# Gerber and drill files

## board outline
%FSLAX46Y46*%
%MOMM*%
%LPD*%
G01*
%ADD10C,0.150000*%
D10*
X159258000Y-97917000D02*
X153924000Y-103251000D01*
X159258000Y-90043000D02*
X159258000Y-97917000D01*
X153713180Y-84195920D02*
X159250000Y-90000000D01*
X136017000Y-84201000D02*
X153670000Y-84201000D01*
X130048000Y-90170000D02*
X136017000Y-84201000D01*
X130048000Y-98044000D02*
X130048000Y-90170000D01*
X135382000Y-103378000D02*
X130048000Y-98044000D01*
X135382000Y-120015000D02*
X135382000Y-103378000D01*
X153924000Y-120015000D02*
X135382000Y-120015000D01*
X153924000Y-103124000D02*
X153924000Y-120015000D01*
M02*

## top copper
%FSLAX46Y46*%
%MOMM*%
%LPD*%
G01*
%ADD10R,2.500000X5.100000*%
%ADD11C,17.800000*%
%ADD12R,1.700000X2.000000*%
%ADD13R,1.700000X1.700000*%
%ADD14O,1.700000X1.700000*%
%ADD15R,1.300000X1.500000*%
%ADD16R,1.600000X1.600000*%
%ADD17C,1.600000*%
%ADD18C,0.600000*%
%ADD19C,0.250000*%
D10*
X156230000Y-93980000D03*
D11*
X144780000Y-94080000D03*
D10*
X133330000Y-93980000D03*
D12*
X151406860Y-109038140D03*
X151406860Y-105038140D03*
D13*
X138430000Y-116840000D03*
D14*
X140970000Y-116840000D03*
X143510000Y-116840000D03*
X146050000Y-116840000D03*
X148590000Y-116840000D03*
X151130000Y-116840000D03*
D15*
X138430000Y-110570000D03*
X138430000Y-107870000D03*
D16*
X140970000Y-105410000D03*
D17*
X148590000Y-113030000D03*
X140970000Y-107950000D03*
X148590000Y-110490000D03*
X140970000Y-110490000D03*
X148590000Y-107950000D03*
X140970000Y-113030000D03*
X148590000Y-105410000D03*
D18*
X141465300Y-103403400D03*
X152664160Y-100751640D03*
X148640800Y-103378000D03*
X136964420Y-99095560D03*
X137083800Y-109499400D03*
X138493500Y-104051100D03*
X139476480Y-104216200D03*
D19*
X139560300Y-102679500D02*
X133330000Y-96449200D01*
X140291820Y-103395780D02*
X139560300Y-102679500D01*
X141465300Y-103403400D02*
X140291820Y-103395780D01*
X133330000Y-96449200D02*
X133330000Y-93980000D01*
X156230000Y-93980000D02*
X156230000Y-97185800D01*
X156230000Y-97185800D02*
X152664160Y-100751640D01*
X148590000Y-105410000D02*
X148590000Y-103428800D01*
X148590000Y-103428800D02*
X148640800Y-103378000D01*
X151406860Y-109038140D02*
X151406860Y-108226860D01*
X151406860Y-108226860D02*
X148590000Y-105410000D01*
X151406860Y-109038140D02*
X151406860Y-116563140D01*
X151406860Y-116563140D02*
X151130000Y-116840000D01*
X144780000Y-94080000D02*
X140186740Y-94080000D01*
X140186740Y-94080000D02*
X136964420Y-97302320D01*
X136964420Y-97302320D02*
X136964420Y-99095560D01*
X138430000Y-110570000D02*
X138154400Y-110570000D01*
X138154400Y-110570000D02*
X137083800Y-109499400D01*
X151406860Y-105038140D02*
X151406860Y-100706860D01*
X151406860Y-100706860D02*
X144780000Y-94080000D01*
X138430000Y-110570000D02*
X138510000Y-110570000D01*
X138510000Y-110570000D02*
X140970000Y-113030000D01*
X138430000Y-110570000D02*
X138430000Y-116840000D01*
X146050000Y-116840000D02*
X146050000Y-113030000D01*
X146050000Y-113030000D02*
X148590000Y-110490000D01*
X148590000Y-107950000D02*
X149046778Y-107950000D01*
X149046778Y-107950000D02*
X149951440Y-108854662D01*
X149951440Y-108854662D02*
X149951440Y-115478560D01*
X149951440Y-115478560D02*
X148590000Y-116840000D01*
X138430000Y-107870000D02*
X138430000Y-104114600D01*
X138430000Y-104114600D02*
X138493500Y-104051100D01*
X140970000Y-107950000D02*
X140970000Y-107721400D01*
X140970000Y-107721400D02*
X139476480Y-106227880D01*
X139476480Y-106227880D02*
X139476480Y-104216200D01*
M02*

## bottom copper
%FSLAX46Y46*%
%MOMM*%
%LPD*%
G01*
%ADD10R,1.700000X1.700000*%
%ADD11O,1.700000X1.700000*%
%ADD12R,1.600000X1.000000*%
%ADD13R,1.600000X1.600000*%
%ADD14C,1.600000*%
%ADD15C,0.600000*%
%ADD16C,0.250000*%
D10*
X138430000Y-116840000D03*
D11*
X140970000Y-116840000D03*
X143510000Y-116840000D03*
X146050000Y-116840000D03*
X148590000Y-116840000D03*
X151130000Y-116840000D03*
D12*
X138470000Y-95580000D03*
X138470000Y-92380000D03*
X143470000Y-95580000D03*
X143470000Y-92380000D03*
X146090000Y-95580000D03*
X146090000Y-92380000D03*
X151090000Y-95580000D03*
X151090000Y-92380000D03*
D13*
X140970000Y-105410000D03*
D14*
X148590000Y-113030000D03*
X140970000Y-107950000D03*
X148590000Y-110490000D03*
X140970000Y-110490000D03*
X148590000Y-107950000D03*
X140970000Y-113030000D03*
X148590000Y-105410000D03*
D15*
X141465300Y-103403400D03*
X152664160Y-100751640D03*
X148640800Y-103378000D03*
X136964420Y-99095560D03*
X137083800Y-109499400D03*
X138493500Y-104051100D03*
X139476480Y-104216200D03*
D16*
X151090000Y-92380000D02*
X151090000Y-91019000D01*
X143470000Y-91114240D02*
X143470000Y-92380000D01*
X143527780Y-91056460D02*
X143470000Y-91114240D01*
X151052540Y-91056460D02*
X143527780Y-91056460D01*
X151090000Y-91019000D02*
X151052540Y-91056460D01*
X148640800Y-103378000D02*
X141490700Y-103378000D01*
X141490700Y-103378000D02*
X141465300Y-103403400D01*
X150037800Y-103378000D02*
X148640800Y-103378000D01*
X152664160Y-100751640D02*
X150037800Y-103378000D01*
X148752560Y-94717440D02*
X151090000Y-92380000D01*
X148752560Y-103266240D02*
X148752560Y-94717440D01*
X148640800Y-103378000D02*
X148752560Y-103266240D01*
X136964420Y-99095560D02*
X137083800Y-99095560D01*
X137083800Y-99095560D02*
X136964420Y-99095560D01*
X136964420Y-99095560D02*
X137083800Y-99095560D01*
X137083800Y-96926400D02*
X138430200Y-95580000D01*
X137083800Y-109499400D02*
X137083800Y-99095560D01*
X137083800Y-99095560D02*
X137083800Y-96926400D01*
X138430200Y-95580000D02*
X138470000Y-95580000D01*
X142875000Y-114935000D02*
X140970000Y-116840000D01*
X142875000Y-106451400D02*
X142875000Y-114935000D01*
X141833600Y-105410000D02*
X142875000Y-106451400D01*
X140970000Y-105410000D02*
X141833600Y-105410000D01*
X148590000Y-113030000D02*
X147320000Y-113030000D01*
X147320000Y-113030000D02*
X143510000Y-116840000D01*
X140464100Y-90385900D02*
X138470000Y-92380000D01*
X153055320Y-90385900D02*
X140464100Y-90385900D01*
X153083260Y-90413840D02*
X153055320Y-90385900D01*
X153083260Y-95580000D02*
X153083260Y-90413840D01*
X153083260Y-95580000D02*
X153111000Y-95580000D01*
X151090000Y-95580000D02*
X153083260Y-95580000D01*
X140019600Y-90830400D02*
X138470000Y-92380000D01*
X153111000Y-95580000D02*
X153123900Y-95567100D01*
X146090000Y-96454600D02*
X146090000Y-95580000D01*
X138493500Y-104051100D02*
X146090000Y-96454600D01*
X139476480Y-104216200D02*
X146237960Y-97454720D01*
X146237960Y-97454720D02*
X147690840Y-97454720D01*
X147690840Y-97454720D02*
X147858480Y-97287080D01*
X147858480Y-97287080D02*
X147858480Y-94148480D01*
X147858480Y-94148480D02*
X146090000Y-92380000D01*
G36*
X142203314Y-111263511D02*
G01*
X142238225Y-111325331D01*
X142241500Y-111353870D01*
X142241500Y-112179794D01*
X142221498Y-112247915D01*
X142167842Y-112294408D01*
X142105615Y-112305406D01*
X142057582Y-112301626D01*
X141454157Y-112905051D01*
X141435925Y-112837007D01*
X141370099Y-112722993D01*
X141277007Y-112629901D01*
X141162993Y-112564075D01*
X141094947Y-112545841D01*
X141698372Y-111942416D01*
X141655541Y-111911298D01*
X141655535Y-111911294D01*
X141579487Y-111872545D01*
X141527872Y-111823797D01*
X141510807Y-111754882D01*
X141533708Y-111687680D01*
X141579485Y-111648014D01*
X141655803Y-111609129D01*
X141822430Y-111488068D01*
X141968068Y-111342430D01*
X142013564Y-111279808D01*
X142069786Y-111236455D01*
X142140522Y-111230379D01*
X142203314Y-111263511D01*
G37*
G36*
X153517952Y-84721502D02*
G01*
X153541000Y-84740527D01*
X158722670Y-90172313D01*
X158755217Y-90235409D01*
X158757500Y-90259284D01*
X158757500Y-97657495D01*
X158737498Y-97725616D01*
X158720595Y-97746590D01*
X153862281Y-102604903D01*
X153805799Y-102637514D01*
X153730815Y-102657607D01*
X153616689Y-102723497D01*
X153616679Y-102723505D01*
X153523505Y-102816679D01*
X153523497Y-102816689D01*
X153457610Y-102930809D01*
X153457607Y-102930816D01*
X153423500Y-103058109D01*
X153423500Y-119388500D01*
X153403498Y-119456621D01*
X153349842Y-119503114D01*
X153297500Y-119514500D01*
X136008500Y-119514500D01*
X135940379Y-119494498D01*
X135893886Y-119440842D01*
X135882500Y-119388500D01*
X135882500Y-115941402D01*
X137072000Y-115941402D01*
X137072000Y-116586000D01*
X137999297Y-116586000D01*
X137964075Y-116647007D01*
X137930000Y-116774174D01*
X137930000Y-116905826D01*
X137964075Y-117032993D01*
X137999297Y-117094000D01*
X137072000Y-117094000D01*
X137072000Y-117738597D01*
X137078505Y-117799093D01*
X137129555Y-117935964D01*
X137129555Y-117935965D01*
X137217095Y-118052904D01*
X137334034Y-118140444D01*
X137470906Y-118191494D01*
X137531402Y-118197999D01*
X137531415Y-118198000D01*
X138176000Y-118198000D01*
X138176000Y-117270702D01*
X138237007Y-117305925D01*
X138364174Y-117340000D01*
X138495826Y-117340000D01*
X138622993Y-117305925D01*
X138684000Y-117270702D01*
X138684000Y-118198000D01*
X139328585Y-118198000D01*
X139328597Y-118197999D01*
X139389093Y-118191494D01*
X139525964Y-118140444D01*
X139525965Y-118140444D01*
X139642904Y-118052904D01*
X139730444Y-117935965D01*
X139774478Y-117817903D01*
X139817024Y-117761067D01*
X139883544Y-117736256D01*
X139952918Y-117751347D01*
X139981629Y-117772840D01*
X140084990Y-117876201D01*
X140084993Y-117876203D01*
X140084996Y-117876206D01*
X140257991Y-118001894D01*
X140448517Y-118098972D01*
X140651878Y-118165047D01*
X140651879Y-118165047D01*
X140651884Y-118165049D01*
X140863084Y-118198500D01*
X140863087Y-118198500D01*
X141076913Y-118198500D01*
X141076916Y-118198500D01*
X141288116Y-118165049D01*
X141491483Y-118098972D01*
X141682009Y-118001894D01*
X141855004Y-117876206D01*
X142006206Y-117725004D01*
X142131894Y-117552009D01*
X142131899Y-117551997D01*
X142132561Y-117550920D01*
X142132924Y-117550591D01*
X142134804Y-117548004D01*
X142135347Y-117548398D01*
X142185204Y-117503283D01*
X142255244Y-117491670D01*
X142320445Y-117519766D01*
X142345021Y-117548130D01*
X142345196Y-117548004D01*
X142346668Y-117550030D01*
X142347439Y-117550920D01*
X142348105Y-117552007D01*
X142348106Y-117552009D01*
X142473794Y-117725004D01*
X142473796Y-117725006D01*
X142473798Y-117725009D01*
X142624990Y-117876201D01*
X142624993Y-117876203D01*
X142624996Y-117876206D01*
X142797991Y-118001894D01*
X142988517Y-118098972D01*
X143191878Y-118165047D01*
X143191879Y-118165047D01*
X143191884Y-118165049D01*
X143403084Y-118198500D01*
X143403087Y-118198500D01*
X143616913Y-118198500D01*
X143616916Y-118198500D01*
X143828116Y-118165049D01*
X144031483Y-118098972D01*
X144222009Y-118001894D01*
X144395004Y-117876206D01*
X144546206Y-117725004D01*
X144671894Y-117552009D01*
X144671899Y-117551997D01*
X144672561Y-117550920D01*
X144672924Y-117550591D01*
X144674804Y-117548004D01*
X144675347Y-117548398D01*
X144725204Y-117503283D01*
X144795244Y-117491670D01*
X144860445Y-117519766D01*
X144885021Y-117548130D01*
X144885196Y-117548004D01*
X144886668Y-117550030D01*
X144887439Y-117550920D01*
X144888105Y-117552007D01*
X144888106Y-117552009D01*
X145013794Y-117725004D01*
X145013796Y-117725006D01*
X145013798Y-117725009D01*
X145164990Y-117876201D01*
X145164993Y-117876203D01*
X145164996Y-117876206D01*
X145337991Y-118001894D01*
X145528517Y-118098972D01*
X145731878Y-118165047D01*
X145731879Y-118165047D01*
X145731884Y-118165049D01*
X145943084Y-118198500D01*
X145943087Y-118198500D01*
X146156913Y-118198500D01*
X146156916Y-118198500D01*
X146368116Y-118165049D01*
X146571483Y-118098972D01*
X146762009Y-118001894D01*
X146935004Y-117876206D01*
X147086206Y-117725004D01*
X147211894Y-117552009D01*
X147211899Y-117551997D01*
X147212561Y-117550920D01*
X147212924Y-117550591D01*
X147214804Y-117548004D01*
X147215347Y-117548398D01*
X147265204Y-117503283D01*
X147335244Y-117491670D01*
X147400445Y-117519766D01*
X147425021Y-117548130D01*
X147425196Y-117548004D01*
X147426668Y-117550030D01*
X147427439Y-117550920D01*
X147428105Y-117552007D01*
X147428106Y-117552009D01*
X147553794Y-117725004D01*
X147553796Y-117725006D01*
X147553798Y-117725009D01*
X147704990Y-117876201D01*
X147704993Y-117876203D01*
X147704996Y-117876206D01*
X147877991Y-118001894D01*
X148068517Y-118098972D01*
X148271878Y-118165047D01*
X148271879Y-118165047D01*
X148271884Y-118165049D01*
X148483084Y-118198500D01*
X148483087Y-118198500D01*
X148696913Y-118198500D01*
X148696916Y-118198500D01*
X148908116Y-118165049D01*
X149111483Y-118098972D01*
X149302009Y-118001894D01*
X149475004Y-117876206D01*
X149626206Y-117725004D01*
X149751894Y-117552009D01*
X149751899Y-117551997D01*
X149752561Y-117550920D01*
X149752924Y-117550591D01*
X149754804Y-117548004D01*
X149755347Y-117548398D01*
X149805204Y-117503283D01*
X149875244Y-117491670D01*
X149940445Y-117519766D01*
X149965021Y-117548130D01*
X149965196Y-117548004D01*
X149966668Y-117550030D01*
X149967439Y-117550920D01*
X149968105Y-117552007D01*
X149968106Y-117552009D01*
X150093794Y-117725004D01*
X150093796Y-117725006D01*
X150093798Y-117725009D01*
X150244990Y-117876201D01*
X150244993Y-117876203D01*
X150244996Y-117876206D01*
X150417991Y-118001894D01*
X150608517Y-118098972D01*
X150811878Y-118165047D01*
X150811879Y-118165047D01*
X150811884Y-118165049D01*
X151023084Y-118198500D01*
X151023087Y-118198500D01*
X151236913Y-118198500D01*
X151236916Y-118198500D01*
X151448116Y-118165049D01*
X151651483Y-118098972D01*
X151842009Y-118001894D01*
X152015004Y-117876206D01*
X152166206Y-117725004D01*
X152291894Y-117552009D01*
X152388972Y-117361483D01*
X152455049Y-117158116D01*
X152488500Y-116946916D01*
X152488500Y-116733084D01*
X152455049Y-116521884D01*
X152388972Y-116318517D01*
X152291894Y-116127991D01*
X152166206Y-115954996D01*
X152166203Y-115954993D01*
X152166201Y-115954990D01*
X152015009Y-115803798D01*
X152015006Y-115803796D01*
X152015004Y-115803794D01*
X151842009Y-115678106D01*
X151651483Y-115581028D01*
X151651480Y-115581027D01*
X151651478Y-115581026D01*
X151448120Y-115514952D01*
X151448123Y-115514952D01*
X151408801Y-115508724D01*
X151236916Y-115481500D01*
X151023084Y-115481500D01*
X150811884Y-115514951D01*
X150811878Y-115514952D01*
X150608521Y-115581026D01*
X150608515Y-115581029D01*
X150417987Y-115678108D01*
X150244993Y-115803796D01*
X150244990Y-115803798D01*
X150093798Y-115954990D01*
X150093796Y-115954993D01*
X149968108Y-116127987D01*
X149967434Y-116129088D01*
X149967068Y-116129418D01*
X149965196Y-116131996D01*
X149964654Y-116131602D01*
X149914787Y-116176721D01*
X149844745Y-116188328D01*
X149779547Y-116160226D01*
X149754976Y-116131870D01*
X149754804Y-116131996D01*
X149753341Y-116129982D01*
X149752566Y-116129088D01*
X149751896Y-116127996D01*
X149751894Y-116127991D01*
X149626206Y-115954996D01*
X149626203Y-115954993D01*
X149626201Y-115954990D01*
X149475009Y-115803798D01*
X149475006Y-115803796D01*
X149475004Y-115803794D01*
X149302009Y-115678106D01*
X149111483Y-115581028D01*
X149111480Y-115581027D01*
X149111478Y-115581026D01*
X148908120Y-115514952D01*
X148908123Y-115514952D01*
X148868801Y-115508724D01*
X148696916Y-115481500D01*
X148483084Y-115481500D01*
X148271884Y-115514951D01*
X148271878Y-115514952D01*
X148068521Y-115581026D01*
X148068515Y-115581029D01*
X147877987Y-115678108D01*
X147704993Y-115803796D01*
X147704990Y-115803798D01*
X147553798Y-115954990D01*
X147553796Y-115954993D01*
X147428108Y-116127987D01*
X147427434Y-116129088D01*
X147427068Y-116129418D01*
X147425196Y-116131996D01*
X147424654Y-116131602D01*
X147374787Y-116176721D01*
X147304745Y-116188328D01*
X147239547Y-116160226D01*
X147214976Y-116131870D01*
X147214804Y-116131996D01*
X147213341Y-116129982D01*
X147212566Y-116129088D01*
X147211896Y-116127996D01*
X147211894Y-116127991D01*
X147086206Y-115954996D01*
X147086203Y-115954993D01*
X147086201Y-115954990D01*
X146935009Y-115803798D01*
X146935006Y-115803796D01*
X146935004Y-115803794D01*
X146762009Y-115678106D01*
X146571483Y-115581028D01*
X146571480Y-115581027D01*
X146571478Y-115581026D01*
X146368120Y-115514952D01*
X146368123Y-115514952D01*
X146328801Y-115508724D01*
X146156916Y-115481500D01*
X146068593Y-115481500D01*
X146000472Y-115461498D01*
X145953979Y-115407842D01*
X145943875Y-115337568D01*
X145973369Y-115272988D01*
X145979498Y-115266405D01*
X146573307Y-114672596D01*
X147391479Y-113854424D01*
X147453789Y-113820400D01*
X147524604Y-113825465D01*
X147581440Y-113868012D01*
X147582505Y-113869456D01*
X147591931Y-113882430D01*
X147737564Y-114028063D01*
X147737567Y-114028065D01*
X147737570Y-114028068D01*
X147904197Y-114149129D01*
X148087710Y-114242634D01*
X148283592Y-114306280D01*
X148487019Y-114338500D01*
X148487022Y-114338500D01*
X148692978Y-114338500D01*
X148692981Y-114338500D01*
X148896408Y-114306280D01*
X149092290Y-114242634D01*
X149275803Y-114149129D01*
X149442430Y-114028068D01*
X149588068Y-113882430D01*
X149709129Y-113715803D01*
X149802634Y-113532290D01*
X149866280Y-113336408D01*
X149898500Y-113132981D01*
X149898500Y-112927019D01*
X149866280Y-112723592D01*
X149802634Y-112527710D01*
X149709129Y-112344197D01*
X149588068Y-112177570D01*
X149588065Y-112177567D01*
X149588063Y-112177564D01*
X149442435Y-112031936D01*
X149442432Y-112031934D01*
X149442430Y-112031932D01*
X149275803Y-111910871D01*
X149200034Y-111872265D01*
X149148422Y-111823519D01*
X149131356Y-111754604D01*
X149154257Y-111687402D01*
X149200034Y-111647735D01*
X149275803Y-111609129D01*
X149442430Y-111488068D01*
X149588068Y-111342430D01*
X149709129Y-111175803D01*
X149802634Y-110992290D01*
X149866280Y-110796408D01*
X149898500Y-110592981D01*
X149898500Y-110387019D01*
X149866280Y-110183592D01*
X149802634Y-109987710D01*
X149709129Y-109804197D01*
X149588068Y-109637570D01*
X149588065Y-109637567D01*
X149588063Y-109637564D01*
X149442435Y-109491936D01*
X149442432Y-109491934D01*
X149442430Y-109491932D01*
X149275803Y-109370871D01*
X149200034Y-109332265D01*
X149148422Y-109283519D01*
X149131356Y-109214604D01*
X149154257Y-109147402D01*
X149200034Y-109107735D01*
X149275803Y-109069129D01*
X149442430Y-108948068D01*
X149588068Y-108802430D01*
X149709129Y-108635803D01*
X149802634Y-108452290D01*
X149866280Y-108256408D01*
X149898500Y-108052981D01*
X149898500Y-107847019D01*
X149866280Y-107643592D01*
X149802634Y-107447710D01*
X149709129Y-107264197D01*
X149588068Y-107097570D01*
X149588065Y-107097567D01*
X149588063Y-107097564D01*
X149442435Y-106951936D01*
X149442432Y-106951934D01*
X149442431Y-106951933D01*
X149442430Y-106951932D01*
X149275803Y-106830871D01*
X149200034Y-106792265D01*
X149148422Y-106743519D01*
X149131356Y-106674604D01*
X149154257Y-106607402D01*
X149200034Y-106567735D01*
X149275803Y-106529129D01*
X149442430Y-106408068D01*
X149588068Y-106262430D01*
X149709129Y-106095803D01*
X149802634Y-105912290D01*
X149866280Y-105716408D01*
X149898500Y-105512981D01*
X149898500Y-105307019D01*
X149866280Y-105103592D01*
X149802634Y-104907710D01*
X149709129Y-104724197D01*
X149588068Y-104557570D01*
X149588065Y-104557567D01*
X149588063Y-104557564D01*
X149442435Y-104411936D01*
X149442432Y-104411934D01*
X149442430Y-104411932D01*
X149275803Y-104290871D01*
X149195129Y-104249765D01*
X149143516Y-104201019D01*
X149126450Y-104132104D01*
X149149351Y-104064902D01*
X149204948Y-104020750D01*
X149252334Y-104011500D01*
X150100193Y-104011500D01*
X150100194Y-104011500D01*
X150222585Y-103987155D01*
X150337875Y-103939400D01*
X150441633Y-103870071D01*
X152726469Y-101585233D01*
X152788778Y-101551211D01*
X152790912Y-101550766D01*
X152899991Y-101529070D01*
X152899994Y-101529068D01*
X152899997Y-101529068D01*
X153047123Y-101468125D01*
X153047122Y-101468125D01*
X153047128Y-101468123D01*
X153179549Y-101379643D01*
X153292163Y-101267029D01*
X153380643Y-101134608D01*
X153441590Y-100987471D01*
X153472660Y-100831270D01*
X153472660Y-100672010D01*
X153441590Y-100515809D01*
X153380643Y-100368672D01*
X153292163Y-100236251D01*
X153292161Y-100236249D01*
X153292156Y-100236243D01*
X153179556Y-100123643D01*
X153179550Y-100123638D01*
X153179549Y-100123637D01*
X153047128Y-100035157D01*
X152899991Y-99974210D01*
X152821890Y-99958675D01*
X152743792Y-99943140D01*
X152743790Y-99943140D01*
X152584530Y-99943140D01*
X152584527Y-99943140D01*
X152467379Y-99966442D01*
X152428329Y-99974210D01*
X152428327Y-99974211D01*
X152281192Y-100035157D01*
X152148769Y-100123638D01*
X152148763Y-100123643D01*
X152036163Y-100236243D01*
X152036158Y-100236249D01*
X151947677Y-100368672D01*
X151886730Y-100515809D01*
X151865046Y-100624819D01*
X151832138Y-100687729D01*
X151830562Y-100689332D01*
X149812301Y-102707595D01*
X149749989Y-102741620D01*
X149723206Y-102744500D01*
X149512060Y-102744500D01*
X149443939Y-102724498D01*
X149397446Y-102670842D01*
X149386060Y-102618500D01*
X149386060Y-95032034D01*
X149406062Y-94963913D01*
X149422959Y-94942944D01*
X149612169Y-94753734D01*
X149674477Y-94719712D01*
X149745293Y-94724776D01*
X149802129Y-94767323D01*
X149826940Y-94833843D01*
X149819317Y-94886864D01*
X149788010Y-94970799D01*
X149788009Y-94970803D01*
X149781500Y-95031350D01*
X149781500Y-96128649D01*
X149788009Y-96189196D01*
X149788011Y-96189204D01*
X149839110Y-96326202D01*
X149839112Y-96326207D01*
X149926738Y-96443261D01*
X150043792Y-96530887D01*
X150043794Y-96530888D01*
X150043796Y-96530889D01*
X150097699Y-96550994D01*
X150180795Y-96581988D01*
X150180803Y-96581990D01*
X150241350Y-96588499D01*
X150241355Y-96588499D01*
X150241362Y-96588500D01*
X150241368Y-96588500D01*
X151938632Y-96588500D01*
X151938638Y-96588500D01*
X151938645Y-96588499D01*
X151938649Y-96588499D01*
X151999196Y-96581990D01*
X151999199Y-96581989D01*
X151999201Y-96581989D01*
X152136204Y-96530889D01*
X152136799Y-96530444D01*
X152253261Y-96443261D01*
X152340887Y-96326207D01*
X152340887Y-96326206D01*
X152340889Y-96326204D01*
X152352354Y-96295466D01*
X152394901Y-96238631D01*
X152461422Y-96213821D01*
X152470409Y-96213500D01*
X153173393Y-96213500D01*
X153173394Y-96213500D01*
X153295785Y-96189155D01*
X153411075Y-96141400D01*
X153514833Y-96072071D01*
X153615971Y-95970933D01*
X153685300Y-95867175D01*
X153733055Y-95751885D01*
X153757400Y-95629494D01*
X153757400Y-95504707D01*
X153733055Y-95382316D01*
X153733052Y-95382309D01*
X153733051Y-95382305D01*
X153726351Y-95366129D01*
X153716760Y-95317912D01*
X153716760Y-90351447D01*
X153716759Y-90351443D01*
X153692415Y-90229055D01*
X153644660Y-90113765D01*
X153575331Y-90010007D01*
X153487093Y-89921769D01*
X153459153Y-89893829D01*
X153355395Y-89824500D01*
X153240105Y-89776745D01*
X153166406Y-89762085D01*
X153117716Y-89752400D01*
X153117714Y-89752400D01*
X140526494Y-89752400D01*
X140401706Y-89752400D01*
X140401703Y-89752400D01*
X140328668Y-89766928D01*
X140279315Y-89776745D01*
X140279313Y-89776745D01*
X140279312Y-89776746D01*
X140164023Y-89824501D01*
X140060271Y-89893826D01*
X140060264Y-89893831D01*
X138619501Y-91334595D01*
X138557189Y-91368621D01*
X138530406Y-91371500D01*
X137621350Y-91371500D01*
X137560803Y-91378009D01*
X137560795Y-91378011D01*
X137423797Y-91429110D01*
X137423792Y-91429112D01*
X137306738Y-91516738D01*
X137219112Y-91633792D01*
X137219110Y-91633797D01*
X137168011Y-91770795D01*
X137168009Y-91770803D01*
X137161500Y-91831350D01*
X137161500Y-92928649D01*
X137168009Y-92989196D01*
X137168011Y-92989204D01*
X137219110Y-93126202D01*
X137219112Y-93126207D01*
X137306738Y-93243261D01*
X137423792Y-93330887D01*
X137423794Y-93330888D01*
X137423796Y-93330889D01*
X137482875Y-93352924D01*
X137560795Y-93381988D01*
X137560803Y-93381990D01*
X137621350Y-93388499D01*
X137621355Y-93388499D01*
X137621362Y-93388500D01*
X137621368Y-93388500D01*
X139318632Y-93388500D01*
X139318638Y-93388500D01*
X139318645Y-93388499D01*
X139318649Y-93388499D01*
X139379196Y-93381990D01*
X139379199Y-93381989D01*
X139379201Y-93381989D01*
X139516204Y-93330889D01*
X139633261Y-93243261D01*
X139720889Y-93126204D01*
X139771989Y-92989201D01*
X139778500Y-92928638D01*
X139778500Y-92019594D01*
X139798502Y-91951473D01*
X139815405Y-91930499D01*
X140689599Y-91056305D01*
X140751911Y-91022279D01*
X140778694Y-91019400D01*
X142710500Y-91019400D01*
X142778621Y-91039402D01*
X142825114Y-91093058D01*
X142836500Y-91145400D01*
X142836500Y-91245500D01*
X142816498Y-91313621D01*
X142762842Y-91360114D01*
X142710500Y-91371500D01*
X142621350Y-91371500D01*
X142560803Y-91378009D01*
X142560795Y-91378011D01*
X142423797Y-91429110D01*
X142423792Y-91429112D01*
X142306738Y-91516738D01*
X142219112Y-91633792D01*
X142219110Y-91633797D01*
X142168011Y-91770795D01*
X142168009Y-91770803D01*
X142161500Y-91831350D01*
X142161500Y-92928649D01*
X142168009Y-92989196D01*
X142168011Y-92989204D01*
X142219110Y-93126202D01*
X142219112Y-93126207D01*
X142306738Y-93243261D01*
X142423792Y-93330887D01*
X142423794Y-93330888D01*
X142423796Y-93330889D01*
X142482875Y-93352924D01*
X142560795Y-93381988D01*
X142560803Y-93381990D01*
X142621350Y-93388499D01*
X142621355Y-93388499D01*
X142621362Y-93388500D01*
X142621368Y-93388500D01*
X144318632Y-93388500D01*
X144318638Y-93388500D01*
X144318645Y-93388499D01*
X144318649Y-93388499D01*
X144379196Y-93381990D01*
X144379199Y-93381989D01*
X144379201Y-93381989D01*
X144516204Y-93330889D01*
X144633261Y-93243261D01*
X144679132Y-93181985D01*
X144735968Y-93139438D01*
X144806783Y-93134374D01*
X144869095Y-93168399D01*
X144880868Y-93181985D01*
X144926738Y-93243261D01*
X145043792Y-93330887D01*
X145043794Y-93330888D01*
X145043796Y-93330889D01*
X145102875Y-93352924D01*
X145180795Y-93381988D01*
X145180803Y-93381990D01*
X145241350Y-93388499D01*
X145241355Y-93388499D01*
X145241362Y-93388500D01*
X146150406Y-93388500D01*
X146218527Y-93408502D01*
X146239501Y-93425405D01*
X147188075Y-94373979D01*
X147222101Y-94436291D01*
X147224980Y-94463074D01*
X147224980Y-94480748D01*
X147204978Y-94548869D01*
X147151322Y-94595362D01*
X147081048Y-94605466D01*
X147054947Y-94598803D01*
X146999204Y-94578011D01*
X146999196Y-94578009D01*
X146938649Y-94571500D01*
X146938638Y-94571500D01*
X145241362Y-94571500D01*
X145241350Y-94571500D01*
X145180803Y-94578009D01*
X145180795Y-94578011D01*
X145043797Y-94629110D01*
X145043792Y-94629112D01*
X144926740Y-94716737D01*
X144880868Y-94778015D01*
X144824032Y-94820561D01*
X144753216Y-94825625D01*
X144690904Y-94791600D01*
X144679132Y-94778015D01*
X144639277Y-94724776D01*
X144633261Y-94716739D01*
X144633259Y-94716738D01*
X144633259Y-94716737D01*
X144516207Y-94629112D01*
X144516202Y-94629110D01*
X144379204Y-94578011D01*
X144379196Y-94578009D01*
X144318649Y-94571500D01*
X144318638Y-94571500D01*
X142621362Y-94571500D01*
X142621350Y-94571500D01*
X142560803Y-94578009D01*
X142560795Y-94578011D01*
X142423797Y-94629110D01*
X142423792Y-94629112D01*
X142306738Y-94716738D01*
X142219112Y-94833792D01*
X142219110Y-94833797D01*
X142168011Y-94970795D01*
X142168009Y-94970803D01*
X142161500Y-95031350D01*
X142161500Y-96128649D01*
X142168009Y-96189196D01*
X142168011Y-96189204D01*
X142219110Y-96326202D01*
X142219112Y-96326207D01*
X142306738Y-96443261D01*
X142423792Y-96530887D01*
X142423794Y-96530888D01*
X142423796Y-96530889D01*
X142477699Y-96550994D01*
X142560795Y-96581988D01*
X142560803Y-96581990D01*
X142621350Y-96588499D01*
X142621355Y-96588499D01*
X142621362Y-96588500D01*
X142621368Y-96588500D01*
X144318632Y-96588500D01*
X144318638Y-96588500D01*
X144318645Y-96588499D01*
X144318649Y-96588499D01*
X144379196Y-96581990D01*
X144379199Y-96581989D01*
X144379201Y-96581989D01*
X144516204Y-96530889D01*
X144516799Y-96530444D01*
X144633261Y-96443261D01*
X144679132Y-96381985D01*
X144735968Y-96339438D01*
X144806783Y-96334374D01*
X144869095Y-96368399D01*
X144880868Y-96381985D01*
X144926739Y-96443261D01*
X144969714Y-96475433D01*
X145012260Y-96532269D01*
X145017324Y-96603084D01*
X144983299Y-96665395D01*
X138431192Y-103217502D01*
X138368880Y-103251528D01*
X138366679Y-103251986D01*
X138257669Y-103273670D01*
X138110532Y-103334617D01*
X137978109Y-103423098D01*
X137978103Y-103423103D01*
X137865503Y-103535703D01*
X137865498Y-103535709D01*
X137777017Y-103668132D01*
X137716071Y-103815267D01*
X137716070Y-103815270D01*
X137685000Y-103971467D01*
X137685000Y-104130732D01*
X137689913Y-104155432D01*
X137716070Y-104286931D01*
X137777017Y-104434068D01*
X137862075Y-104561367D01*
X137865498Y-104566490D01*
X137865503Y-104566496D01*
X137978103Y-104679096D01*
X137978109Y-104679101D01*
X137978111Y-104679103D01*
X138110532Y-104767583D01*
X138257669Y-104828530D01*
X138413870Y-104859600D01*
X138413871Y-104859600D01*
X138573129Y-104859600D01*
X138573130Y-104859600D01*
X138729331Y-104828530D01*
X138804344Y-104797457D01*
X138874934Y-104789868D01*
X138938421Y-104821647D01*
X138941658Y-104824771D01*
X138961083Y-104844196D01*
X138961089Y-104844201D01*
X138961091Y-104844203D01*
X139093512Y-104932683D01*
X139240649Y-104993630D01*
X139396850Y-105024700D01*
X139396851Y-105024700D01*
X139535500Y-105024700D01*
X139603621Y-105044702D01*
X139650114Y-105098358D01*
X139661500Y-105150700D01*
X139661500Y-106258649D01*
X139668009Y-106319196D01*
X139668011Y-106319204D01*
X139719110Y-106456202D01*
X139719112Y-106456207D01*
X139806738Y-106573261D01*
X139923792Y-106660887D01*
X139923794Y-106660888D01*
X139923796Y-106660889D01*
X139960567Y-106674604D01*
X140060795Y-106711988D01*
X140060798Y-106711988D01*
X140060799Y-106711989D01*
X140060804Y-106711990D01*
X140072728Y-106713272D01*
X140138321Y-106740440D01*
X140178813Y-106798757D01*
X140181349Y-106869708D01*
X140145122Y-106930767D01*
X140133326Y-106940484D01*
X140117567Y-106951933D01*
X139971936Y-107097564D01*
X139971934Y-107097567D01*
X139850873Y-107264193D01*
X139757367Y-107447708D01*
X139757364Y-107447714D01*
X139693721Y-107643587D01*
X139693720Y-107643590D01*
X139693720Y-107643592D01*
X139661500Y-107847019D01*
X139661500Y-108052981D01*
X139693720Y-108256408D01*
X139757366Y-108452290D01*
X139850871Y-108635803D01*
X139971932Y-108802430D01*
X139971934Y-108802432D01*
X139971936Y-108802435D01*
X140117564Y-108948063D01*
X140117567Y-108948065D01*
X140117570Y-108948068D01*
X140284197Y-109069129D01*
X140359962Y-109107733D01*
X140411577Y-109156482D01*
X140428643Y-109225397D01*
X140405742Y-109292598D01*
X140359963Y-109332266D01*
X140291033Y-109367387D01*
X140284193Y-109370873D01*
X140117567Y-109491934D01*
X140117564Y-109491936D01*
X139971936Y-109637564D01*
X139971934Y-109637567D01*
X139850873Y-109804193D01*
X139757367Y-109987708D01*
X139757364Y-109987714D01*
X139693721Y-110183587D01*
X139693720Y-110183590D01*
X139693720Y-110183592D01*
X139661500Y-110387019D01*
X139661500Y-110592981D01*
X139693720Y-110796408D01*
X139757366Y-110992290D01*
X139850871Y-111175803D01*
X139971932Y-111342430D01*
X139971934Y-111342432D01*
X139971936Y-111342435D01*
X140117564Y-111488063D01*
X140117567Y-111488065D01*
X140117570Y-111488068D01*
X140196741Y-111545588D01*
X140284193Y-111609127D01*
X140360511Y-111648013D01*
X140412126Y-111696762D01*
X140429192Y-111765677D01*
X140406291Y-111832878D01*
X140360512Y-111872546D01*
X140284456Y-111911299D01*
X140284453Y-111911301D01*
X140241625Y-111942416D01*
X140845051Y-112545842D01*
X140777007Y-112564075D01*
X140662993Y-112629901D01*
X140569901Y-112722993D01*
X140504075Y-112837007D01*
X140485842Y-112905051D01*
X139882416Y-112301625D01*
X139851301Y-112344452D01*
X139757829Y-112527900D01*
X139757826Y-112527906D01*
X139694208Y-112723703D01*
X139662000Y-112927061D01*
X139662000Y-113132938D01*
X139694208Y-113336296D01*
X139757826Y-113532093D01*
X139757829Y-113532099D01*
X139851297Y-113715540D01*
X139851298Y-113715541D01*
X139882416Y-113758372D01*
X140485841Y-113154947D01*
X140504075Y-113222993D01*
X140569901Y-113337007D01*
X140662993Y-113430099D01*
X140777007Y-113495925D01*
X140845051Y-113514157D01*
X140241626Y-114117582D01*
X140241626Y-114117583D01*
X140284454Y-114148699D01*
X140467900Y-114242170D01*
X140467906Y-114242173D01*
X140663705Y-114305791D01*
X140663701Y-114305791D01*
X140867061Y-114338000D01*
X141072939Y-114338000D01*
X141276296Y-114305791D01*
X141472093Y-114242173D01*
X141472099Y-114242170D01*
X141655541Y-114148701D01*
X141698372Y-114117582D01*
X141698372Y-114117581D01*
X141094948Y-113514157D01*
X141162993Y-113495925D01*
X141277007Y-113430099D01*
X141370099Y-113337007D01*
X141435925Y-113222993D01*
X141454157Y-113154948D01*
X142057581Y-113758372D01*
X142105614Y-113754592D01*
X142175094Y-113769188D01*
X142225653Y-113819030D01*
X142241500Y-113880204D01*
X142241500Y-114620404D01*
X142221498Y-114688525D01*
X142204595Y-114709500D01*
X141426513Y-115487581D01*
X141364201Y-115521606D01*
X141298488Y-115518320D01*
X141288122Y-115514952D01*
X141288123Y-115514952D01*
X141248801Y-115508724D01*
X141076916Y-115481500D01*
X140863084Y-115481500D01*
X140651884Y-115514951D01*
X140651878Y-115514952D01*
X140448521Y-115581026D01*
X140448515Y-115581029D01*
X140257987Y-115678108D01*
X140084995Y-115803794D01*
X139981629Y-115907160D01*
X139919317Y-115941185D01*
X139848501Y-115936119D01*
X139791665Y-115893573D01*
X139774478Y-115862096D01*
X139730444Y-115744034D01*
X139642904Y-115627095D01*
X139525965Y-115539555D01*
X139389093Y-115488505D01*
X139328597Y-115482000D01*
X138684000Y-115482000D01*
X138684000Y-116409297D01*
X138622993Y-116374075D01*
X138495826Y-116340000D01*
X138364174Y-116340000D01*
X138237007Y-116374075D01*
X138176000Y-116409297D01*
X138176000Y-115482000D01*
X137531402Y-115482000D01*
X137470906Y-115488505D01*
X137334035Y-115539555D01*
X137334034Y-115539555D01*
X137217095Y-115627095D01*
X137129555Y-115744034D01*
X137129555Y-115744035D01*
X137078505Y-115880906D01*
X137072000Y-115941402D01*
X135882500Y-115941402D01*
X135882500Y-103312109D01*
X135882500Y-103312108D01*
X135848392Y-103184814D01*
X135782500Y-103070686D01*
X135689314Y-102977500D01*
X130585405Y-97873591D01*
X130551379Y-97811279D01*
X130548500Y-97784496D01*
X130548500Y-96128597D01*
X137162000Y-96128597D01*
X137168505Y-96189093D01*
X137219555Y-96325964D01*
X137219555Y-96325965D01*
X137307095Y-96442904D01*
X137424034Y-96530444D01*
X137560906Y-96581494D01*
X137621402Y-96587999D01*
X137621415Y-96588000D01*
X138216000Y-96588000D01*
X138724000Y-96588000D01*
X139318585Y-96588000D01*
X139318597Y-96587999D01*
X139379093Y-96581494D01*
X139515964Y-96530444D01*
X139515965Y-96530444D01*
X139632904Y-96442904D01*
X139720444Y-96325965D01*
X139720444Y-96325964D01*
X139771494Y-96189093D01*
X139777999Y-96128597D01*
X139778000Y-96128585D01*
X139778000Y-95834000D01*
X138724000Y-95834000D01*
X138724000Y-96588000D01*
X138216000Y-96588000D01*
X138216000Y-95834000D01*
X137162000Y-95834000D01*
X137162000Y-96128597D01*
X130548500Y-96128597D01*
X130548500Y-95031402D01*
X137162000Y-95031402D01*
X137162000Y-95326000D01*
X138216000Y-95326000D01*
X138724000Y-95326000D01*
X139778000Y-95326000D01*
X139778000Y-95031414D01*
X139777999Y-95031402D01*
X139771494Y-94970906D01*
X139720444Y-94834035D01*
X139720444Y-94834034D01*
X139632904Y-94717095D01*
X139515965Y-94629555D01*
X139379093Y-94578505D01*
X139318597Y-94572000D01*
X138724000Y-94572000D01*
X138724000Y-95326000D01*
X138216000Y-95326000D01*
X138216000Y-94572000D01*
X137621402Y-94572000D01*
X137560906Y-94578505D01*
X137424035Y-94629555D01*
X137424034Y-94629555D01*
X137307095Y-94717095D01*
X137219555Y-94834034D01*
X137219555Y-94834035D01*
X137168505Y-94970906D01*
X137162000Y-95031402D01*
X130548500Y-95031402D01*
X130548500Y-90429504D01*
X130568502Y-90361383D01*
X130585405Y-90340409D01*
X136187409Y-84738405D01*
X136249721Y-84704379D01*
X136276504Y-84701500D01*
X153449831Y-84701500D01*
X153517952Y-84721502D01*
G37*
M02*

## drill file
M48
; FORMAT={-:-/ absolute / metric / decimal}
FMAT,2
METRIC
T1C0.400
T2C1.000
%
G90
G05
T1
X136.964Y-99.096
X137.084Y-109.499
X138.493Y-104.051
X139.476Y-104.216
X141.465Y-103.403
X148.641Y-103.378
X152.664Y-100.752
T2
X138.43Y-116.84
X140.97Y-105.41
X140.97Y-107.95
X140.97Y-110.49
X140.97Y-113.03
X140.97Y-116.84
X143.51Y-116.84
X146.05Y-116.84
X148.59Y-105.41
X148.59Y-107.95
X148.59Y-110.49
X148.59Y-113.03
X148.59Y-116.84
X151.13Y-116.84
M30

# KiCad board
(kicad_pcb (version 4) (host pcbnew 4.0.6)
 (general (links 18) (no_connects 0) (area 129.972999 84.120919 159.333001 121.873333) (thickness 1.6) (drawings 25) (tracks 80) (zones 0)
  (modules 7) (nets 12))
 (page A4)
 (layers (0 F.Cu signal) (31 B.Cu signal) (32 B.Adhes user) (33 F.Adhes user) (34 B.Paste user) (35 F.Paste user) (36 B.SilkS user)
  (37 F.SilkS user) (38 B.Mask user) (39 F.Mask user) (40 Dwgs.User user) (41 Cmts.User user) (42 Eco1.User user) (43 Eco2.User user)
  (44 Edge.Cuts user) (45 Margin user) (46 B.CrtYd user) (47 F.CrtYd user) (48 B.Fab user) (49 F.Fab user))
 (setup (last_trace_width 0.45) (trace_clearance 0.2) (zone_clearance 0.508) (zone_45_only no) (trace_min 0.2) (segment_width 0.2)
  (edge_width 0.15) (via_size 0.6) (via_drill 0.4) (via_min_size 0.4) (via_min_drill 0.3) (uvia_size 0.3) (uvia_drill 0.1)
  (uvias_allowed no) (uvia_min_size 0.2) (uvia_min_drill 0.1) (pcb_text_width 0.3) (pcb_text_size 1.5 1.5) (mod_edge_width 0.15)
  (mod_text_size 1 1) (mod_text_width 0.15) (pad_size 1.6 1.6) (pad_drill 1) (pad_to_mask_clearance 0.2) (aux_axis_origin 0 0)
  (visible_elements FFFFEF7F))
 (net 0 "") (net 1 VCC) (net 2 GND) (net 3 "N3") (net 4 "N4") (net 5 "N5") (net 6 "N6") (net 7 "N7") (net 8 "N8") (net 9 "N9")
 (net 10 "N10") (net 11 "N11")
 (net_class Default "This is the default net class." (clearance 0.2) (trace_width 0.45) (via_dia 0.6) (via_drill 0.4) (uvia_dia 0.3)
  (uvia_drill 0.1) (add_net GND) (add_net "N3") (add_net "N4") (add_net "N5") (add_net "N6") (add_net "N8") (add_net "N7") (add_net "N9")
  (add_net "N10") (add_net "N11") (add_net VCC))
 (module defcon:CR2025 (layer F.Cu) (at 144.78 93.98)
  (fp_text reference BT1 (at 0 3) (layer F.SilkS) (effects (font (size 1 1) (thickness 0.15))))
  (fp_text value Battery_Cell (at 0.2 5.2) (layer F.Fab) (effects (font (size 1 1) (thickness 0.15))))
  (pad 1 smd rect (at 11.45 0) (size 2.5 5.1) (layers F.Cu F.Paste F.Mask) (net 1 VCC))
  (pad 2 smd circle (at 0 0.1) (size 17.8 17.8) (layers F.Cu F.Paste F.Mask) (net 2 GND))
  (pad 1 smd rect (at -11.45 0) (size 2.5 5.1) (layers F.Cu F.Paste F.Mask) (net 1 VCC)))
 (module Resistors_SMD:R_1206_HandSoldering (layer F.Cu) (at 151.40686 107.03814 90)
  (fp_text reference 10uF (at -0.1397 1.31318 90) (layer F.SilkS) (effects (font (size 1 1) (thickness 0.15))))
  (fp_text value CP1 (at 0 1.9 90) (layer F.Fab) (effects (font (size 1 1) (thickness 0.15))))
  (pad 1 smd rect (at -2 0 90) (size 2 1.7) (layers F.Cu F.Paste F.Mask) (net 1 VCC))
  (pad 2 smd rect (at 2 0 90) (size 2 1.7) (layers F.Cu F.Paste F.Mask) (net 2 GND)))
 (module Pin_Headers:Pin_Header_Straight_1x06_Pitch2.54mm (layer F.Cu) (at 138.43 116.84 90)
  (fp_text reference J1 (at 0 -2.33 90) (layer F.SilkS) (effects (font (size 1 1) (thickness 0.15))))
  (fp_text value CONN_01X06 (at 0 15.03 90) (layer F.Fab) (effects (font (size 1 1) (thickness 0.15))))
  (pad 1 thru_hole rect (at 0 0 90) (size 1.7 1.7) (drill 1) (layers *.Cu *.Mask) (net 2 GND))
  (pad 2 thru_hole oval (at 0 2.54 90) (size 1.7 1.7) (drill 1) (layers *.Cu *.Mask) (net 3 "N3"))
  (pad 3 thru_hole oval (at 0 5.08 90) (size 1.7 1.7) (drill 1) (layers *.Cu *.Mask) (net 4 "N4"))
  (pad 4 thru_hole oval (at 0 7.62 90) (size 1.7 1.7) (drill 1) (layers *.Cu *.Mask) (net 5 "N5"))
  (pad 5 thru_hole oval (at 0 10.16 90) (size 1.7 1.7) (drill 1) (layers *.Cu *.Mask) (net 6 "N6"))
  (pad 6 thru_hole oval (at 0 12.7 90) (size 1.7 1.7) (drill 1) (layers *.Cu *.Mask) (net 1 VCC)))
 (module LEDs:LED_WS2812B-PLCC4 (layer B.Cu) (at 140.97 93.98 180)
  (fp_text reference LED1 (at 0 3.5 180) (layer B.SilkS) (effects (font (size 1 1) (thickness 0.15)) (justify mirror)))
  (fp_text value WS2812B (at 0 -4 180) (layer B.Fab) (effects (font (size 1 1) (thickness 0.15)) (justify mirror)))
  (pad 3 smd rect (at 2.5 -1.6 180) (size 1.6 1) (layers B.Cu B.Paste B.Mask) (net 2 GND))
  (pad 4 smd rect (at 2.5 1.6 180) (size 1.6 1) (layers B.Cu B.Paste B.Mask) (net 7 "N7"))
  (pad 2 smd rect (at -2.5 -1.6 180) (size 1.6 1) (layers B.Cu B.Paste B.Mask) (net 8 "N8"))
  (pad 1 smd rect (at -2.5 1.6 180) (size 1.6 1) (layers B.Cu B.Paste B.Mask) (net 1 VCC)))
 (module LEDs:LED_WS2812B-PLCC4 (layer B.Cu) (at 148.59 93.98 180)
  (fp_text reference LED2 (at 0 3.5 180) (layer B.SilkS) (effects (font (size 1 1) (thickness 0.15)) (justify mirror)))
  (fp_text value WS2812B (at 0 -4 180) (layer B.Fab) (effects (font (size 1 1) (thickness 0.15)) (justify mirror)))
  (pad 3 smd rect (at 2.5 -1.6 180) (size 1.6 1) (layers B.Cu B.Paste B.Mask) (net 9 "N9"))
  (pad 4 smd rect (at 2.5 1.6 180) (size 1.6 1) (layers B.Cu B.Paste B.Mask) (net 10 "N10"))
  (pad 2 smd rect (at -2.5 -1.6 180) (size 1.6 1) (layers B.Cu B.Paste B.Mask) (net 7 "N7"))
  (pad 1 smd rect (at -2.5 1.6 180) (size 1.6 1) (layers B.Cu B.Paste B.Mask) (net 1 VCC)))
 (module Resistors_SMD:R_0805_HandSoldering (layer F.Cu) (at 138.43 109.22 90)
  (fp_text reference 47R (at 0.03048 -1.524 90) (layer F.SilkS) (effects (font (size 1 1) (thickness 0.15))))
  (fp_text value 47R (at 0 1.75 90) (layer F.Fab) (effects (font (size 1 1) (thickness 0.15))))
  (pad 1 smd rect (at -1.35 0 90) (size 1.5 1.3) (layers F.Cu F.Paste F.Mask) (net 2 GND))
  (pad 2 smd rect (at 1.35 0 90) (size 1.5 1.3) (layers F.Cu F.Paste F.Mask) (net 9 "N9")))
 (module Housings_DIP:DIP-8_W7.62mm (layer F.Cu) (at 140.97 105.41)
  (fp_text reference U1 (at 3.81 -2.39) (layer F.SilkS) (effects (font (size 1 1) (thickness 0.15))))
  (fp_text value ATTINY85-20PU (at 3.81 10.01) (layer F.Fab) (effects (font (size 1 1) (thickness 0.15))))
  (pad 1 thru_hole rect (at 0 0) (size 1.6 1.6) (drill 1) (layers *.Cu *.Mask) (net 3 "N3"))
  (pad 5 thru_hole circle (at 7.62 7.62) (size 1.6 1.6) (drill 1) (layers *.Cu *.Mask) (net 4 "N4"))
  (pad 2 thru_hole circle (at 0 2.54) (size 1.6 1.6) (drill 1) (layers *.Cu *.Mask) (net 10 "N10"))
  (pad 6 thru_hole circle (at 7.62 5.08) (size 1.6 1.6) (drill 1) (layers *.Cu *.Mask) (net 5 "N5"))
  (pad 3 thru_hole circle (at 0 5.08) (size 1.6 1.6) (drill 1) (layers *.Cu *.Mask) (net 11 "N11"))
  (pad 7 thru_hole circle (at 7.62 2.54) (size 1.6 1.6) (drill 1) (layers *.Cu *.Mask) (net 6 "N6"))
  (pad 4 thru_hole circle (at 0 7.62) (size 1.6 1.6) (drill 1) (layers *.Cu *.Mask) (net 2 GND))
  (pad 8 thru_hole circle (at 7.62 0) (size 1.6 1.6) (drill 1) (layers *.Cu *.Mask) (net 1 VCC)))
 (gr_line (start 159.258 97.917) (end 153.924 103.251) (angle 90) (layer Edge.Cuts) (width 0.15))
 (gr_line (start 159.258 90.043) (end 159.258 97.917) (angle 90) (layer Edge.Cuts) (width 0.15))
 (gr_line (start 153.71318 84.19592) (end 159.25 90) (angle 90) (layer Edge.Cuts) (width 0.15))
 (gr_line (start 136.017 84.201) (end 153.67 84.201) (angle 90) (layer Edge.Cuts) (width 0.15))
 (gr_line (start 130.048 90.17) (end 136.017 84.201) (angle 90) (layer Edge.Cuts) (width 0.15))
 (gr_line (start 130.048 98.044) (end 130.048 90.17) (angle 90) (layer Edge.Cuts) (width 0.15))
 (gr_line (start 135.382 103.378) (end 130.048 98.044) (angle 90) (layer Edge.Cuts) (width 0.15))
 (gr_line (start 135.382 120.015) (end 135.382 103.378) (angle 90) (layer Edge.Cuts) (width 0.15))
 (gr_line (start 153.924 120.015) (end 135.382 120.015) (angle 90) (layer Edge.Cuts) (width 0.15))
 (gr_line (start 153.924 103.124) (end 153.924 120.015) (angle 90) (layer Edge.Cuts) (width 0.15))
 (segment (start 151.09 92.38) (end 151.09 91.019) (width 0.25) (layer B.Cu) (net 1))
 (segment (start 143.47 91.11424) (end 143.47 92.38) (width 0.25) (layer B.Cu) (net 1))
 (segment (start 143.52778 91.05646) (end 143.47 91.11424) (width 0.25) (layer B.Cu) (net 1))
 (segment (start 151.05254 91.05646) (end 143.52778 91.05646) (width 0.25) (layer B.Cu) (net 1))
 (segment (start 151.09 91.019) (end 151.05254 91.05646) (width 0.25) (layer B.Cu) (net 1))
 (segment (start 148.6408 103.378) (end 141.4907 103.378) (width 0.25) (layer B.Cu) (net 1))
 (segment (start 139.5603 102.6795) (end 133.33 96.4492) (width 0.25) (layer F.Cu) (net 1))
 (segment (start 140.29182 103.39578) (end 139.5603 102.6795) (width 0.25) (layer F.Cu) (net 1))
 (segment (start 141.4653 103.4034) (end 140.29182 103.39578) (width 0.25) (layer F.Cu) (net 1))
 (via (at 141.4653 103.4034) (size 0.6) (drill 0.4) (layers F.Cu B.Cu) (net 1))
 (segment (start 141.4907 103.378) (end 141.4653 103.4034) (width 0.25) (layer B.Cu) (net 1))
 (segment (start 133.33 96.4492) (end 133.33 93.98) (width 0.25) (layer F.Cu) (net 1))
 (segment (start 156.23 93.98) (end 156.23 97.1858) (width 0.25) (layer F.Cu) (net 1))
 (segment (start 150.0378 103.378) (end 148.6408 103.378) (width 0.25) (layer B.Cu) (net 1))
 (segment (start 152.66416 100.75164) (end 150.0378 103.378) (width 0.25) (layer B.Cu) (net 1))
 (via (at 152.66416 100.75164) (size 0.6) (drill 0.4) (layers F.Cu B.Cu) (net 1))
 (segment (start 156.23 97.1858) (end 152.66416 100.75164) (width 0.25) (layer F.Cu) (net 1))
 (segment (start 148.59 105.41) (end 148.59 103.4288) (width 0.25) (layer F.Cu) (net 1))
 (segment (start 148.75256 94.71744) (end 151.09 92.38) (width 0.25) (layer B.Cu) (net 1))
 (segment (start 148.75256 103.26624) (end 148.75256 94.71744) (width 0.25) (layer B.Cu) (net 1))
 (segment (start 148.6408 103.378) (end 148.75256 103.26624) (width 0.25) (layer B.Cu) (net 1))
 (via (at 148.6408 103.378) (size 0.6) (drill 0.4) (layers F.Cu B.Cu) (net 1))
 (segment (start 148.59 103.4288) (end 148.6408 103.378) (width 0.25) (layer F.Cu) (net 1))
 (segment (start 151.40686 109.03814) (end 151.40686 108.22686) (width 0.25) (layer F.Cu) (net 1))
 (segment (start 151.40686 108.22686) (end 148.59 105.41) (width 0.25) (layer F.Cu) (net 1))
 (segment (start 151.40686 109.03814) (end 151.40686 116.56314) (width 0.25) (layer F.Cu) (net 1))
 (segment (start 151.40686 116.56314) (end 151.13 116.84) (width 0.25) (layer F.Cu) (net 1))
 (via (at 136.96442 99.09556) (size 0.6) (drill 0.4) (layers F.Cu B.Cu) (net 2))
 (segment (start 144.78 94.08) (end 140.18674 94.08) (width 0.25) (layer F.Cu) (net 2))
 (segment (start 140.18674 94.08) (end 136.96442 97.30232) (width 0.25) (layer F.Cu) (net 2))
 (segment (start 136.96442 97.30232) (end 136.96442 99.09556) (width 0.25) (layer F.Cu) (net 2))
 (segment (start 136.96442 99.09556) (end 137.0838 99.09556) (width 0.25) (layer B.Cu) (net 2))
 (segment (start 137.0838 99.09556) (end 136.96442 99.09556) (width 0.25) (layer B.Cu) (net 2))
 (segment (start 136.96442 99.09556) (end 137.0838 99.09556) (width 0.25) (layer B.Cu) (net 2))
 (segment (start 138.43 110.57) (end 138.1544 110.57) (width 0.25) (layer F.Cu) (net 2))
 (segment (start 138.1544 110.57) (end 137.0838 109.4994) (width 0.25) (layer F.Cu) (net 2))
 (segment (start 137.0838 96.9264) (end 138.4302 95.58) (width 0.25) (layer B.Cu) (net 2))
 (segment (start 137.0838 109.4994) (end 137.0838 99.09556) (width 0.25) (layer B.Cu) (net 2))
 (segment (start 137.0838 99.09556) (end 137.0838 96.9264) (width 0.25) (layer B.Cu) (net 2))
 (via (at 137.0838 109.4994) (size 0.6) (drill 0.4) (layers F.Cu B.Cu) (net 2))
 (segment (start 138.4302 95.58) (end 138.47 95.58) (width 0.25) (layer B.Cu) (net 2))
 (segment (start 151.40686 105.03814) (end 151.40686 100.70686) (width 0.25) (layer F.Cu) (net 2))
 (segment (start 151.40686 100.70686) (end 144.78 94.08) (width 0.25) (layer F.Cu) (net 2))
 (segment (start 138.43 110.57) (end 138.51 110.57) (width 0.25) (layer F.Cu) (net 2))
 (segment (start 138.51 110.57) (end 140.97 113.03) (width 0.25) (layer F.Cu) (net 2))
 (segment (start 138.43 110.57) (end 138.43 116.84) (width 0.25) (layer F.Cu) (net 2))
 (segment (start 142.875 114.935) (end 140.97 116.84) (width 0.25) (layer B.Cu) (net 3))
 (segment (start 142.875 106.4514) (end 142.875 114.935) (width 0.25) (layer B.Cu) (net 3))
 (segment (start 141.8336 105.41) (end 142.875 106.4514) (width 0.25) (layer B.Cu) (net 3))
 (segment (start 140.97 105.41) (end 141.8336 105.41) (width 0.25) (layer B.Cu) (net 3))
 (segment (start 148.59 113.03) (end 147.32 113.03) (width 0.25) (layer B.Cu) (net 4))
 (segment (start 147.32 113.03) (end 143.51 116.84) (width 0.25) (layer B.Cu) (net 4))
 (segment (start 146.05 116.84) (end 146.05 113.03) (width 0.25) (layer F.Cu) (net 5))
 (segment (start 146.05 113.03) (end 148.59 110.49) (width 0.25) (layer F.Cu) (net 5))
 (segment (start 148.59 107.95) (end 149.046778 107.95) (width 0.25) (layer F.Cu) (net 6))
 (segment (start 149.046778 107.95) (end 149.95144 108.854662) (width 0.25) (layer F.Cu) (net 6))
 (segment (start 149.95144 108.854662) (end 149.95144 115.47856) (width 0.25) (layer F.Cu) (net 6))
 (segment (start 149.95144 115.47856) (end 148.59 116.84) (width 0.25) (layer F.Cu) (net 6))
 (segment (start 140.4641 90.3859) (end 138.47 92.38) (width 0.25) (layer B.Cu) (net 7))
 (segment (start 153.05532 90.3859) (end 140.4641 90.3859) (width 0.25) (layer B.Cu) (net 7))
 (segment (start 153.08326 90.41384) (end 153.05532 90.3859) (width 0.25) (layer B.Cu) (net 7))
 (segment (start 153.08326 95.58) (end 153.08326 90.41384) (width 0.25) (layer B.Cu) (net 7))
 (segment (start 153.08326 95.58) (end 153.111 95.58) (width 0.25) (layer B.Cu) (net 7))
 (segment (start 151.09 95.58) (end 153.08326 95.58) (width 0.25) (layer B.Cu) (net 7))
 (segment (start 140.0196 90.8304) (end 138.47 92.38) (width 0.25) (layer B.Cu) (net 7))
 (segment (start 153.111 95.58) (end 153.1239 95.5671) (width 0.25) (layer B.Cu) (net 7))
 (segment (start 138.43 107.87) (end 138.43 104.1146) (width 0.25) (layer F.Cu) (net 9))
 (segment (start 146.09 96.4546) (end 146.09 95.58) (width 0.25) (layer B.Cu) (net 9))
 (segment (start 138.4935 104.0511) (end 146.09 96.4546) (width 0.25) (layer B.Cu) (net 9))
 (via (at 138.4935 104.0511) (size 0.6) (drill 0.4) (layers F.Cu B.Cu) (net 9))
 (segment (start 138.43 104.1146) (end 138.4935 104.0511) (width 0.25) (layer F.Cu) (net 9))
 (segment (start 140.97 107.95) (end 140.97 107.7214) (width 0.25) (layer F.Cu) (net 10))
 (segment (start 140.97 107.7214) (end 139.47648 106.22788) (width 0.25) (layer F.Cu) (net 10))
 (segment (start 139.47648 106.22788) (end 139.47648 104.2162) (width 0.25) (layer F.Cu) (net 10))
 (via (at 139.47648 104.2162) (size 0.6) (drill 0.4) (layers F.Cu B.Cu) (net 10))
 (segment (start 139.47648 104.2162) (end 146.23796 97.45472) (width 0.25) (layer B.Cu) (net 10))
 (segment (start 146.23796 97.45472) (end 147.69084 97.45472) (width 0.25) (layer B.Cu) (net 10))
 (segment (start 147.69084 97.45472) (end 147.85848 97.28708) (width 0.25) (layer B.Cu) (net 10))
 (segment (start 147.85848 97.28708) (end 147.85848 94.14848) (width 0.25) (layer B.Cu) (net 10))
 (segment (start 147.85848 94.14848) (end 146.09 92.38) (width 0.25) (layer B.Cu) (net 10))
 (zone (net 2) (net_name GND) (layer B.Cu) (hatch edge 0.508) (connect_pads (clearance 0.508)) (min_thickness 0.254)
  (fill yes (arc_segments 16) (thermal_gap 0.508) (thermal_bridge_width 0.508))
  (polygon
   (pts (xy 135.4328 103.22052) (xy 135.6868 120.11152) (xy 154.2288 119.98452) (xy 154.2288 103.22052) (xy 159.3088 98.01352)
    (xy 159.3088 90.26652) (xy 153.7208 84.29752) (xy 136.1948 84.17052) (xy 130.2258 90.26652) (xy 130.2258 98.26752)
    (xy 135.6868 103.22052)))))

